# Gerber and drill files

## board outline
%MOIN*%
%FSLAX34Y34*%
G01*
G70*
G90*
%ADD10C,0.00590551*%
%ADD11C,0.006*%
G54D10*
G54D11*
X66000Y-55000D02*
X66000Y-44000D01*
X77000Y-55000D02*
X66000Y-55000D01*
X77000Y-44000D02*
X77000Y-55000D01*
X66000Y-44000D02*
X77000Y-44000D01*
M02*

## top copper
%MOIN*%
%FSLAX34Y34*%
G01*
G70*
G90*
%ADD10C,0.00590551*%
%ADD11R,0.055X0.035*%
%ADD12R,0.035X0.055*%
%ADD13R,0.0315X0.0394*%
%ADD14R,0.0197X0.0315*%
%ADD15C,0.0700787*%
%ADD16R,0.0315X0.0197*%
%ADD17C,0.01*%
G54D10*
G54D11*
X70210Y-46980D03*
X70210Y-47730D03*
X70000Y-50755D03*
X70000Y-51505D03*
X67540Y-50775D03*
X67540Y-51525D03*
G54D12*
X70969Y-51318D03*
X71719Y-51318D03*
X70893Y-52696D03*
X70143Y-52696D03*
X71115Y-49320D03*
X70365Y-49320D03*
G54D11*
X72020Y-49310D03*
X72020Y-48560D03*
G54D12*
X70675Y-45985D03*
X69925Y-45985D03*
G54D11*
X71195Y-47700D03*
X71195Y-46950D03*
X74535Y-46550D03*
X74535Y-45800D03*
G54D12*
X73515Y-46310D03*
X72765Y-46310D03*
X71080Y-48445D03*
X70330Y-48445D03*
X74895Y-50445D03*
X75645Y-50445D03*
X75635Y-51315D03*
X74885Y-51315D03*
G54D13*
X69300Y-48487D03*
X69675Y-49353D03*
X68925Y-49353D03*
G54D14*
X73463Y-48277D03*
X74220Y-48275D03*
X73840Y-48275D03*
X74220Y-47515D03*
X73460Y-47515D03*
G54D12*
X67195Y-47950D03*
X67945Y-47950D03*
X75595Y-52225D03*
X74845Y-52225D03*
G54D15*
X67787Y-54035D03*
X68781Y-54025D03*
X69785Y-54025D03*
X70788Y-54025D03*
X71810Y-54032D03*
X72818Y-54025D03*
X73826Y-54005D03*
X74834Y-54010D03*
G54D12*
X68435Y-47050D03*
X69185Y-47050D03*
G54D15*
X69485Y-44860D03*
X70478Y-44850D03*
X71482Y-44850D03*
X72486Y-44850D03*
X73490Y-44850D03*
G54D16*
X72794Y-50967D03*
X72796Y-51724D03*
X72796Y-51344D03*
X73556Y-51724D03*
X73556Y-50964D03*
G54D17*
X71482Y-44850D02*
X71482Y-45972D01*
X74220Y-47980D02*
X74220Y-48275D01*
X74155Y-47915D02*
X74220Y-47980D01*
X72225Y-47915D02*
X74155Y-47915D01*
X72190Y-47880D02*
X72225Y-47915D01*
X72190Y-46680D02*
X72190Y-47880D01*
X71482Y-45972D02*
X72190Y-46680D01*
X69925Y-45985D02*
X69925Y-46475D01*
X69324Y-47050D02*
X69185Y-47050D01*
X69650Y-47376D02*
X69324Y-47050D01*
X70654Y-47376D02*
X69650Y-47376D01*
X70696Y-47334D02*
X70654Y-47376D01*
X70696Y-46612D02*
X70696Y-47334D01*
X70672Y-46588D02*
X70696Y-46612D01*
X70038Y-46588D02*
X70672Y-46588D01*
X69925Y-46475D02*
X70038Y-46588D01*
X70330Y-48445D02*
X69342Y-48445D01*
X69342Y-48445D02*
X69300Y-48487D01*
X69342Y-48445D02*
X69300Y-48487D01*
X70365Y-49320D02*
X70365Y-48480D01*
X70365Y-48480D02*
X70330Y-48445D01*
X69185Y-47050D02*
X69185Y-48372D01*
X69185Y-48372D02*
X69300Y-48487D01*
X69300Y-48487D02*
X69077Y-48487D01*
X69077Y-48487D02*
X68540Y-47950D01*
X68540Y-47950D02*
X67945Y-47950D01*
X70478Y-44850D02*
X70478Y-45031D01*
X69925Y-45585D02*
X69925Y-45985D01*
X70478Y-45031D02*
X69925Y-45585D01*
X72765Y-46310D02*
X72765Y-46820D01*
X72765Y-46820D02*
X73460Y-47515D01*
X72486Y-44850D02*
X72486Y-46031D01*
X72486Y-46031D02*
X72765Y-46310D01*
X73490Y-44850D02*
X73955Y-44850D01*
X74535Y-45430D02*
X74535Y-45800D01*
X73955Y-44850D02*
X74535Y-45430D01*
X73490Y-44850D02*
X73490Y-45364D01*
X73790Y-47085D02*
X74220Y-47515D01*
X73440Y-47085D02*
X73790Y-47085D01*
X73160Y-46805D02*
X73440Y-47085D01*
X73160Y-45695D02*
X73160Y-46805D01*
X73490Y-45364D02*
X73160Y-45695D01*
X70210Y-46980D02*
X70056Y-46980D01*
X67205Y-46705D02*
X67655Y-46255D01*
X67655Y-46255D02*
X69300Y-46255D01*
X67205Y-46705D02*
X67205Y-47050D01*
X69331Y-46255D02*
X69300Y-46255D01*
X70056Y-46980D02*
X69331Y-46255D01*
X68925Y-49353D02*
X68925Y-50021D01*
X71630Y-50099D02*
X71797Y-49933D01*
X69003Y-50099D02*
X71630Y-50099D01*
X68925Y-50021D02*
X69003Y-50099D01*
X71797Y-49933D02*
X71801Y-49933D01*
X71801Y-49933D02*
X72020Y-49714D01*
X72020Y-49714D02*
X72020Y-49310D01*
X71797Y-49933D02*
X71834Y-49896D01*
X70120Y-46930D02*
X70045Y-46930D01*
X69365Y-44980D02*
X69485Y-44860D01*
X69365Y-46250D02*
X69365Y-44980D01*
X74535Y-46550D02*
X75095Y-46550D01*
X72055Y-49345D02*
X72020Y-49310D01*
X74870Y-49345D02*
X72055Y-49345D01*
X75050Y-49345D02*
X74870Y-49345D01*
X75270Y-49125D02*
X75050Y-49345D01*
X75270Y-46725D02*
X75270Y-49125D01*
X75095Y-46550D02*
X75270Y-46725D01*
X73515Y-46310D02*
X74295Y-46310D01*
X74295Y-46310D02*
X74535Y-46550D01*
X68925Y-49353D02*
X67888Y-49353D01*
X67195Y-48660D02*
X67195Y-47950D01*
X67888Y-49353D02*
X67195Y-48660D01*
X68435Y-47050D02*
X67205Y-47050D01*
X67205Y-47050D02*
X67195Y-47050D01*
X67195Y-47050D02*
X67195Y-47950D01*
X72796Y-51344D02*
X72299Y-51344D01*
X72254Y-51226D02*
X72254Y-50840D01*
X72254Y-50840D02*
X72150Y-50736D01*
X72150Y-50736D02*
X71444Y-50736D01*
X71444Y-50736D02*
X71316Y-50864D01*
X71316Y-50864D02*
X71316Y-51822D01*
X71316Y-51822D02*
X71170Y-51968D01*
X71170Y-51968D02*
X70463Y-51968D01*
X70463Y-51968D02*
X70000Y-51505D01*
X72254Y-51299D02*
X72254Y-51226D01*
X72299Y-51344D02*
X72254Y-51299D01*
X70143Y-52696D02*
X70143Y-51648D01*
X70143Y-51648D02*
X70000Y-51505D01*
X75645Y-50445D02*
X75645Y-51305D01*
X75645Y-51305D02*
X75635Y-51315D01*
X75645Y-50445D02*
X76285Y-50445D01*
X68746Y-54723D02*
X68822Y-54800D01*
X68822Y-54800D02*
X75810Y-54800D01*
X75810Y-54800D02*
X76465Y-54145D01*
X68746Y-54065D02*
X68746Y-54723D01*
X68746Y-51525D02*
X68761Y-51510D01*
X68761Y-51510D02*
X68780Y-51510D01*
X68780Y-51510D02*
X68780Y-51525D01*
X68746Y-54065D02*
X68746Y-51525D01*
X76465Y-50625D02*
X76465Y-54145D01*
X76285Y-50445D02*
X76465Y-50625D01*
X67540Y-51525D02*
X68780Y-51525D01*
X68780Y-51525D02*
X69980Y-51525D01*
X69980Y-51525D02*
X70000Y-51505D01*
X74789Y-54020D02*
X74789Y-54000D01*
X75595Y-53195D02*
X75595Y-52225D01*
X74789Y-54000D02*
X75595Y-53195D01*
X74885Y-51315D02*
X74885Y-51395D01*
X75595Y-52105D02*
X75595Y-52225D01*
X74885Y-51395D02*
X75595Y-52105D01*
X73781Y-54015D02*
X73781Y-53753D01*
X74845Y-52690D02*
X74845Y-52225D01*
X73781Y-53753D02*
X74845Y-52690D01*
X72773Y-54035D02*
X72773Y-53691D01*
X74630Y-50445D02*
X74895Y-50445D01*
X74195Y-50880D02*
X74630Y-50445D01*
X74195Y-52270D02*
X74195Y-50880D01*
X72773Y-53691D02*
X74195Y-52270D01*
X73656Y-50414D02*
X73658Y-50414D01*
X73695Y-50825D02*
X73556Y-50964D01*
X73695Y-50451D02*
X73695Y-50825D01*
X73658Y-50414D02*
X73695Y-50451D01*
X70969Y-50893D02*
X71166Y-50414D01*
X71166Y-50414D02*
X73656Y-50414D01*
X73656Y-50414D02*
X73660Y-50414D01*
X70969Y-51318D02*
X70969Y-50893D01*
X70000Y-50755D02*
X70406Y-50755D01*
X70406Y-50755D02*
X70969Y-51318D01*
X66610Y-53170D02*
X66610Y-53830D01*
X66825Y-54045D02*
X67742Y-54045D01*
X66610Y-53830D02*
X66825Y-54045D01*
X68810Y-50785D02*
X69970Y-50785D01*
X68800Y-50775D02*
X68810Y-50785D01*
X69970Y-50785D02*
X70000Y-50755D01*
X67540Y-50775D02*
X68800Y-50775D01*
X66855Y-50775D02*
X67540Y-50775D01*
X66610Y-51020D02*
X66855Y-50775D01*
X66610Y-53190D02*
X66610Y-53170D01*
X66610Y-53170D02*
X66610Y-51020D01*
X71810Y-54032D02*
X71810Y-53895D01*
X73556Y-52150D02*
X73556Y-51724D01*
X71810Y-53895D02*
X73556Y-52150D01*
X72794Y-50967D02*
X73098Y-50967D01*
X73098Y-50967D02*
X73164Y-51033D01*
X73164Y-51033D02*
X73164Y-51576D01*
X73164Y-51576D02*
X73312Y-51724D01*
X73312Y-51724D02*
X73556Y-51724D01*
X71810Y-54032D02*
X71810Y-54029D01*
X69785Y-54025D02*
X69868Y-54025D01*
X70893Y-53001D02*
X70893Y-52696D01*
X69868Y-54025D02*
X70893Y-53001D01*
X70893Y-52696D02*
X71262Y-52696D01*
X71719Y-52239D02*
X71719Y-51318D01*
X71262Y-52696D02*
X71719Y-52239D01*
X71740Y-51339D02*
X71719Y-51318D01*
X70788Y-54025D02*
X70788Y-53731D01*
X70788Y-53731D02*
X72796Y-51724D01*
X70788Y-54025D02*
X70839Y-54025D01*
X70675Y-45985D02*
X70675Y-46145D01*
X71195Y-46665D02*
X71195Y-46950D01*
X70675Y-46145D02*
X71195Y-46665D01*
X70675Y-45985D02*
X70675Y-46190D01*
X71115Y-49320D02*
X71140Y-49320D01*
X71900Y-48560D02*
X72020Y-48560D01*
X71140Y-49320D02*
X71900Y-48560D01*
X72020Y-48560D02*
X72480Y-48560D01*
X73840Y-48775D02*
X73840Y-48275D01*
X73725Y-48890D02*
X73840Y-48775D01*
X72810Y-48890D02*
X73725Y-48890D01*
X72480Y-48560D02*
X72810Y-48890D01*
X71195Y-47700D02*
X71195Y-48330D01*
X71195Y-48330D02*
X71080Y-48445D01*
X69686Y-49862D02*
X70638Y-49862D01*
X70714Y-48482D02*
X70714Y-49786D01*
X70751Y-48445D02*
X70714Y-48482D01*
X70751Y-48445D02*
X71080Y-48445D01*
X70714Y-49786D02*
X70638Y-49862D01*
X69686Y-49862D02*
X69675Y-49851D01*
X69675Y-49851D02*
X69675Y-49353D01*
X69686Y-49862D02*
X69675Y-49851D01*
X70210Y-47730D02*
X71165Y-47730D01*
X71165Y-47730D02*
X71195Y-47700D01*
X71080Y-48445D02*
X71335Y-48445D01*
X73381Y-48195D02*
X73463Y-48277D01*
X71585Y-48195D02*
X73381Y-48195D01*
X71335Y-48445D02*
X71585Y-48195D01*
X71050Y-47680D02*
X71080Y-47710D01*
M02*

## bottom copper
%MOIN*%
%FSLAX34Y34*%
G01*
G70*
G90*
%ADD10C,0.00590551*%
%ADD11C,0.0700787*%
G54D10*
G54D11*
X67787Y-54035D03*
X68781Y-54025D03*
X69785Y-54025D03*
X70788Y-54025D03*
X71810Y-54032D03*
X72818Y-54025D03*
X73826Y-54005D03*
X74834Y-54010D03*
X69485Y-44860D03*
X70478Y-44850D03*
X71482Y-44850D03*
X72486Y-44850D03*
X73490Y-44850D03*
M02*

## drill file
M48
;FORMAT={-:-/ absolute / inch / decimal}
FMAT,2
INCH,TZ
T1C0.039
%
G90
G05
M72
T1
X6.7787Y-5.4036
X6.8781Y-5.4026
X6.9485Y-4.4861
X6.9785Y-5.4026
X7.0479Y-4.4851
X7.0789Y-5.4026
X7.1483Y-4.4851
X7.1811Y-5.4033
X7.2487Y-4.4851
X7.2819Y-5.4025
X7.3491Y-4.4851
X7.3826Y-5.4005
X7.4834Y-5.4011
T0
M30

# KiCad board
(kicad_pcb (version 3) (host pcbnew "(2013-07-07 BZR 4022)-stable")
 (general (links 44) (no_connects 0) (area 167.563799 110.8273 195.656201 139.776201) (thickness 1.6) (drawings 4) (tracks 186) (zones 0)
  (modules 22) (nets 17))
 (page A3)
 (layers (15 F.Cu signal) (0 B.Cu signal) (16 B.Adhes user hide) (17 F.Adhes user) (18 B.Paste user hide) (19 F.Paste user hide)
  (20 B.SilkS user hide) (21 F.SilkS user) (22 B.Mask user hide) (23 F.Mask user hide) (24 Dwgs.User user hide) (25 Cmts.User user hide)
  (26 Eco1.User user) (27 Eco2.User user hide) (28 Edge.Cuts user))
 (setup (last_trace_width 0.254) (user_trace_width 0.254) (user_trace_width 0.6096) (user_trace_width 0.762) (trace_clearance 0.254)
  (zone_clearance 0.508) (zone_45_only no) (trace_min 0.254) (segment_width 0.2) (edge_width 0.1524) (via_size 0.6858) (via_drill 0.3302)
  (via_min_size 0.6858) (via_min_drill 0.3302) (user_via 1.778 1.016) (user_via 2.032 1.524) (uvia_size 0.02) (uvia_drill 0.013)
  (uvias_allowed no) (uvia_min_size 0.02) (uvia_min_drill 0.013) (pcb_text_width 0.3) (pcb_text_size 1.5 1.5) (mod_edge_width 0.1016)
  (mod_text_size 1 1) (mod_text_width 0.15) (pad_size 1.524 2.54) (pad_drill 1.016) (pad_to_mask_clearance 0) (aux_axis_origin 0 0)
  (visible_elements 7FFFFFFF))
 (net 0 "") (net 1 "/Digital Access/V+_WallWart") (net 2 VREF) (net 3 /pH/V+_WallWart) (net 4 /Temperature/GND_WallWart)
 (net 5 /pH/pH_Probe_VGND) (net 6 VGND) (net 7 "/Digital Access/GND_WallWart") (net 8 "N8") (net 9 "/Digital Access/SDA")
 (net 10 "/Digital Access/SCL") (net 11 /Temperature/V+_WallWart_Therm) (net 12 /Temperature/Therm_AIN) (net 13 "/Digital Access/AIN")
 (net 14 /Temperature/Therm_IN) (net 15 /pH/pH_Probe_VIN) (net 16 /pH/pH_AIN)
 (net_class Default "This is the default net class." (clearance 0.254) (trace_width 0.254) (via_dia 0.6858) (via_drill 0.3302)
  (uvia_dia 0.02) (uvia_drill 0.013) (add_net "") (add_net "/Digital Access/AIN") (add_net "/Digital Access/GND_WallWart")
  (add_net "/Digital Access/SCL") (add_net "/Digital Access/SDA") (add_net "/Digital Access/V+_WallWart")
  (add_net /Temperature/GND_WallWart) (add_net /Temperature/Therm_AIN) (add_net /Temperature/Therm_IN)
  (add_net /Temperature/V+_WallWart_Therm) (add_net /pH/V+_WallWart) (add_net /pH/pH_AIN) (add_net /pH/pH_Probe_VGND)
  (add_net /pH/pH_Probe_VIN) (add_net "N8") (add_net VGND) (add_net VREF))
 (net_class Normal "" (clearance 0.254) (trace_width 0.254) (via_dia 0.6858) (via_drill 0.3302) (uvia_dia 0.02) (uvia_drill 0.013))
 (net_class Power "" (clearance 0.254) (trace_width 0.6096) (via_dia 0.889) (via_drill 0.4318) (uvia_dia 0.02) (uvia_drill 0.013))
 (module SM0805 (layer F.Cu) (at 178.3334 120.2817 270)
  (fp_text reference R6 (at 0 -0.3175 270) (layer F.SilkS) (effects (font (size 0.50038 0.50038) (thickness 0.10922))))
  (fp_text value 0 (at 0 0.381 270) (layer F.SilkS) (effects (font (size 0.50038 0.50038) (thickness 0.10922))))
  (pad 1 smd rect (at -0.9525 0 270) (size 0.889 1.397) (layers F.Cu F.Paste F.Mask) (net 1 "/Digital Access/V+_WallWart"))
  (pad 2 smd rect (at 0.9525 0 270) (size 0.889 1.397) (layers F.Cu F.Paste F.Mask) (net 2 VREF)))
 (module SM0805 (layer F.Cu) (at 177.8 129.8702 270)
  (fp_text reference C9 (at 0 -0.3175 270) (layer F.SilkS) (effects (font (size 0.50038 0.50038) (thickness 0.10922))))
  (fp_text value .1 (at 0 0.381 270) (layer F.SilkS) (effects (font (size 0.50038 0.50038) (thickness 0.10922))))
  (pad 1 smd rect (at -0.9525 0 270) (size 0.889 1.397) (layers F.Cu F.Paste F.Mask) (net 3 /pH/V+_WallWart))
  (pad 2 smd rect (at 0.9525 0 270) (size 0.889 1.397) (layers F.Cu F.Paste F.Mask) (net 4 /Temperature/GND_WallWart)))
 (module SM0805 (layer F.Cu) (at 171.5516 129.921 270)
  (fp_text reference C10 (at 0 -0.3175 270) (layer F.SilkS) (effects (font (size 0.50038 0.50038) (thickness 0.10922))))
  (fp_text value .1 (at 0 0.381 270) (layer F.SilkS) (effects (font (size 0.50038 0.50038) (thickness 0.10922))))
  (pad 1 smd rect (at -0.9525 0 270) (size 0.889 1.397) (layers F.Cu F.Paste F.Mask) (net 3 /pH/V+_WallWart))
  (pad 2 smd rect (at 0.9525 0 270) (size 0.889 1.397) (layers F.Cu F.Paste F.Mask) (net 4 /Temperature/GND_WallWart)))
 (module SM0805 (layer F.Cu) (at 181.21376 130.34772)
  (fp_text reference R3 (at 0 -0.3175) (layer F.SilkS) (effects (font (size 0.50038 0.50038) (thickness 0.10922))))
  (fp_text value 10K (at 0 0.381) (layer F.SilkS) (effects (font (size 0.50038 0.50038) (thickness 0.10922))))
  (pad 1 smd rect (at -0.9525 0) (size 0.889 1.397) (layers F.Cu F.Paste F.Mask) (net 3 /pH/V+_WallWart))
  (pad 2 smd rect (at 0.9525 0) (size 0.889 1.397) (layers F.Cu F.Paste F.Mask) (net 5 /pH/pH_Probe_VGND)))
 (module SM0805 (layer F.Cu) (at 179.11572 133.84784 180)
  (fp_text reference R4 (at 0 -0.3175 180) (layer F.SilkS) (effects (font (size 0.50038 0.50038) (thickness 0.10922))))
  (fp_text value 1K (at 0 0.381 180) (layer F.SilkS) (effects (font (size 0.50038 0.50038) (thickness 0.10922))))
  (pad 1 smd rect (at -0.9525 0 180) (size 0.889 1.397) (layers F.Cu F.Paste F.Mask) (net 5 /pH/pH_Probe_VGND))
  (pad 2 smd rect (at 0.9525 0 180) (size 0.889 1.397) (layers F.Cu F.Paste F.Mask) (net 4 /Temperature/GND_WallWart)))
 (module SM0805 (layer F.Cu) (at 179.6796 125.2728 180)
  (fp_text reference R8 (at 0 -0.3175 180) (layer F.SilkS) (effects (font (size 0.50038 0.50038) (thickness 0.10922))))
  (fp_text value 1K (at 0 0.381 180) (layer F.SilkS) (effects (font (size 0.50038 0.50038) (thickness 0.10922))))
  (pad 1 smd rect (at -0.9525 0 180) (size 0.889 1.397) (layers F.Cu F.Paste F.Mask) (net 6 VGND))
  (pad 2 smd rect (at 0.9525 0 180) (size 0.889 1.397) (layers F.Cu F.Paste F.Mask) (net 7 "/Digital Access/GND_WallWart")))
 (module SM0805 (layer F.Cu) (at 182.9308 124.2949 90)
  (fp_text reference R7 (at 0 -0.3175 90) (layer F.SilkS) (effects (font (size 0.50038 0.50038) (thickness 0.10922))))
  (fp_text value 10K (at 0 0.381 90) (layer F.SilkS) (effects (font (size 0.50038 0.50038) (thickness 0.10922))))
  (pad 1 smd rect (at -0.9525 0 90) (size 0.889 1.397) (layers F.Cu F.Paste F.Mask) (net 1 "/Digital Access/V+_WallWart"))
  (pad 2 smd rect (at 0.9525 0 90) (size 0.889 1.397) (layers F.Cu F.Paste F.Mask) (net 6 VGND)))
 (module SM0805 (layer F.Cu) (at 178.562 116.8019 180)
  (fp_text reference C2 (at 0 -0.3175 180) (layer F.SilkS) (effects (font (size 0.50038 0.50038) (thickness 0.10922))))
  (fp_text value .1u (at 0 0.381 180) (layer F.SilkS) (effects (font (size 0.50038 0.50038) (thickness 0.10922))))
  (pad 1 smd rect (at -0.9525 0 180) (size 0.889 1.397) (layers F.Cu F.Paste F.Mask) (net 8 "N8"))
  (pad 2 smd rect (at 0.9525 0 180) (size 0.889 1.397) (layers F.Cu F.Paste F.Mask) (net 7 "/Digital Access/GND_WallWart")))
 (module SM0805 (layer F.Cu) (at 180.8353 120.2055 90)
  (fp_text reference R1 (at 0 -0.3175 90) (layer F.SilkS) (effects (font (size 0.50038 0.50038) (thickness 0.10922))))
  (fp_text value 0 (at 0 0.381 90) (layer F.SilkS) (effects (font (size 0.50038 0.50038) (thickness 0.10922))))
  (pad 1 smd rect (at -0.9525 0 90) (size 0.889 1.397) (layers F.Cu F.Paste F.Mask) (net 2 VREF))
  (pad 2 smd rect (at 0.9525 0 90) (size 0.889 1.397) (layers F.Cu F.Paste F.Mask) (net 8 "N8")))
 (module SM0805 (layer F.Cu) (at 189.3189 117.2845 90)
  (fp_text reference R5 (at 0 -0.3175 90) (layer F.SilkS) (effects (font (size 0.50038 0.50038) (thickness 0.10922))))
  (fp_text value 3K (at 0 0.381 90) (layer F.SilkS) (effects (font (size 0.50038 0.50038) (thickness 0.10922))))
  (pad 1 smd rect (at -0.9525 0 90) (size 0.889 1.397) (layers F.Cu F.Paste F.Mask) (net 1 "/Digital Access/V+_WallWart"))
  (pad 2 smd rect (at 0.9525 0 90) (size 0.889 1.397) (layers F.Cu F.Paste F.Mask) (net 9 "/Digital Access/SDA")))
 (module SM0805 (layer F.Cu) (at 185.7756 117.6274 180)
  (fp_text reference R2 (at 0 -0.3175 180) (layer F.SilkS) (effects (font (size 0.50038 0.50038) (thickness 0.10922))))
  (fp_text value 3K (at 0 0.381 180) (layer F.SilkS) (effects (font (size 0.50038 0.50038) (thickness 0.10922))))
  (pad 1 smd rect (at -0.9525 0 180) (size 0.889 1.397) (layers F.Cu F.Paste F.Mask) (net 1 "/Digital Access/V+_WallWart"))
  (pad 2 smd rect (at 0.9525 0 180) (size 0.889 1.397) (layers F.Cu F.Paste F.Mask) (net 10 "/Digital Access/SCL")))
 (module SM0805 (layer F.Cu) (at 179.5907 123.0503 180)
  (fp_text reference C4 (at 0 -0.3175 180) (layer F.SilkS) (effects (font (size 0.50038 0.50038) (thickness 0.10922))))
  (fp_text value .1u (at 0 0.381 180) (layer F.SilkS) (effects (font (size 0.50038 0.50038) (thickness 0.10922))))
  (pad 1 smd rect (at -0.9525 0 180) (size 0.889 1.397) (layers F.Cu F.Paste F.Mask) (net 2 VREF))
  (pad 2 smd rect (at 0.9525 0 180) (size 0.889 1.397) (layers F.Cu F.Paste F.Mask) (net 7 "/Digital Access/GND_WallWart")))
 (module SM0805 (layer F.Cu) (at 191.1858 128.1303)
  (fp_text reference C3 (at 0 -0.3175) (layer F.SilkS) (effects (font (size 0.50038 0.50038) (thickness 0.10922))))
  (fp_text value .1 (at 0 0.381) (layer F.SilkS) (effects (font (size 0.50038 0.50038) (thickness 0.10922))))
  (pad 1 smd rect (at -0.9525 0) (size 0.889 1.397) (layers F.Cu F.Paste F.Mask) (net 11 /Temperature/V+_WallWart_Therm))
  (pad 2 smd rect (at 0.9525 0) (size 0.889 1.397) (layers F.Cu F.Paste F.Mask) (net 4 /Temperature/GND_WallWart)))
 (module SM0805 (layer F.Cu) (at 191.1604 130.3401 180)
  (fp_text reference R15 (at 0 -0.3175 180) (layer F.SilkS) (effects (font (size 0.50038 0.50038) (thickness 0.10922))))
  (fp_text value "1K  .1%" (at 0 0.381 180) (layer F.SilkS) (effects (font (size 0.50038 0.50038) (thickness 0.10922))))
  (pad 1 smd rect (at -0.9525 0 180) (size 0.889 1.397) (layers F.Cu F.Paste F.Mask) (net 4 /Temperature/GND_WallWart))
  (pad 2 smd rect (at 0.9525 0 180) (size 0.889 1.397) (layers F.Cu F.Paste F.Mask) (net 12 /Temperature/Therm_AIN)))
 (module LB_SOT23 (layer F.Cu) (at 176.022 124.2568)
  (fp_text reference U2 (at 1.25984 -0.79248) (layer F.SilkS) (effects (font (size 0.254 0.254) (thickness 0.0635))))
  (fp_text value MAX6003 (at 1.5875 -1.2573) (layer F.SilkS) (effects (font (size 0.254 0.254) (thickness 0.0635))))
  (pad 3 smd rect (at 0 -1.09982) (size 0.8001 1.00076) (layers F.Cu F.Paste F.Mask) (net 7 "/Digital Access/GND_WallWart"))
  (pad 2 smd rect (at 0.9525 1.09982) (size 0.8001 1.00076) (layers F.Cu F.Paste F.Mask) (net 2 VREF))
  (pad 1 smd rect (at -0.9525 1.09982) (size 0.8001 1.00076) (layers F.Cu F.Paste F.Mask) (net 1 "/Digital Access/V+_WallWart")))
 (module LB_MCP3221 (layer F.Cu) (at 186.5884 122.5423)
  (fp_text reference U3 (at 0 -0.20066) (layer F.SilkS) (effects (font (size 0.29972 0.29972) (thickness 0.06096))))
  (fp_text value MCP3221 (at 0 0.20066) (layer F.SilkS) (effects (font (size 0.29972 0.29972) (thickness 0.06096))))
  (pad 1 smd rect (at 0.00762 0.08128) (size 0.50038 0.8001) (layers F.Cu F.Paste F.Mask) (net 2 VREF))
  (pad 3 smd rect (at 1.9304 0.0762) (size 0.50038 0.8001) (layers F.Cu F.Paste F.Mask) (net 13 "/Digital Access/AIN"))
  (pad 2 smd rect (at 0.9652 0.0762) (size 0.50038 0.8001) (layers F.Cu F.Paste F.Mask) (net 6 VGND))
  (pad 4 smd rect (at 1.9304 -1.8542) (size 0.50038 0.8001) (layers F.Cu F.Paste F.Mask) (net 9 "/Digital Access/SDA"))
  (pad 5 smd rect (at 0 -1.8542) (size 0.50038 0.8001) (layers F.Cu F.Paste F.Mask) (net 10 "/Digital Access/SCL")))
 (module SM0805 (layer F.Cu) (at 171.6278 121.793)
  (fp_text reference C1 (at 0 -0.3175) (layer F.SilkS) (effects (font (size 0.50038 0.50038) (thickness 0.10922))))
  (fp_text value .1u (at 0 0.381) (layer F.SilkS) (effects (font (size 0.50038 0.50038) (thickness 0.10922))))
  (pad 1 smd rect (at -0.9525 0) (size 0.889 1.397) (layers F.Cu F.Paste F.Mask) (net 1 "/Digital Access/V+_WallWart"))
  (pad 2 smd rect (at 0.9525 0) (size 0.889 1.397) (layers F.Cu F.Paste F.Mask) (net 7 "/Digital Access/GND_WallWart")))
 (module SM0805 (layer F.Cu) (at 191.0588 132.6515 180)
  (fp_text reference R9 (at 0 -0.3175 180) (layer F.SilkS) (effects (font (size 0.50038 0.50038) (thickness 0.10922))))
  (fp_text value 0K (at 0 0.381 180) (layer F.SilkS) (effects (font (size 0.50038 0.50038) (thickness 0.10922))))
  (pad 1 smd rect (at -0.9525 0 180) (size 0.889 1.397) (layers F.Cu F.Paste F.Mask) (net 12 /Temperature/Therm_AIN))
  (pad 2 smd rect (at 0.9525 0 180) (size 0.889 1.397) (layers F.Cu F.Paste F.Mask) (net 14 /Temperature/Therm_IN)))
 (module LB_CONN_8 (layer F.Cu) (at 177.2793 137.2108)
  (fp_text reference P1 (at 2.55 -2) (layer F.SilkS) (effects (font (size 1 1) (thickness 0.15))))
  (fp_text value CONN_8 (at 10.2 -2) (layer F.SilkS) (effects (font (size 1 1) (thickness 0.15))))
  (pad 1 thru_hole circle (at -5.1 0.04) (size 1.78 1.78) (drill 1) (layers *.Cu *.Mask F.SilkS) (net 3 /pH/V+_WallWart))
  (pad 2 thru_hole circle (at -2.5754 0.0146) (size 1.78 1.78) (drill 1) (layers *.Cu *.Mask F.SilkS) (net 4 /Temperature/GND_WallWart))
  (pad 3 thru_hole circle (at -0.0254 0.0146) (size 1.78 1.78) (drill 1) (layers *.Cu *.Mask F.SilkS) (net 5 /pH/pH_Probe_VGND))
  (pad 4 thru_hole circle (at 2.5246 0.0146) (size 1.78 1.78) (drill 1) (layers *.Cu *.Mask F.SilkS) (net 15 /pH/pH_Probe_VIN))
  (pad 5 thru_hole circle (at 5.12 0.033) (size 1.78 1.78) (drill 1) (layers *.Cu *.Mask F.SilkS) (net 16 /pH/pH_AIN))
  (pad 6 thru_hole circle (at 7.68 0.013) (size 1.78 1.78) (drill 1) (layers *.Cu *.Mask F.SilkS) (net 11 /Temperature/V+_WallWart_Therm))
  (pad 7 thru_hole circle (at 10.24 -0.038) (size 1.78 1.78) (drill 1) (layers *.Cu *.Mask F.SilkS) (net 14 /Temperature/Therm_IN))
  (pad 8 thru_hole circle (at 12.8 -0.023) (size 1.78 1.78) (drill 1) (layers *.Cu *.Mask F.SilkS) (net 12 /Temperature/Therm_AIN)))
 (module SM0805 (layer F.Cu) (at 174.7774 119.507)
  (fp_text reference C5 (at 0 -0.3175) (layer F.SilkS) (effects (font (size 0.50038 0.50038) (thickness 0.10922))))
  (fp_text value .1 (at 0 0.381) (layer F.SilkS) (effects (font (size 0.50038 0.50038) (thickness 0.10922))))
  (pad 1 smd rect (at -0.9525 0) (size 0.889 1.397) (layers F.Cu F.Paste F.Mask) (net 1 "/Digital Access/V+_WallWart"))
  (pad 2 smd rect (at 0.9525 0) (size 0.889 1.397) (layers F.Cu F.Paste F.Mask) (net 7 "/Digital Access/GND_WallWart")))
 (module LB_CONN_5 (layer F.Cu) (at 176.4919 113.9063)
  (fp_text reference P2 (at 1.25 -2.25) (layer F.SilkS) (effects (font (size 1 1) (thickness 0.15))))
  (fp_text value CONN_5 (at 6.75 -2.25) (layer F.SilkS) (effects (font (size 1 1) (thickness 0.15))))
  (pad 1 thru_hole circle (at 0 0.04) (size 1.78 1.78) (drill 1) (layers *.Cu *.Mask F.SilkS) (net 1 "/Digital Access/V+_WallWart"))
  (pad 2 thru_hole circle (at 2.5246 0.0146) (size 1.78 1.78) (drill 1) (layers *.Cu *.Mask F.SilkS) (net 7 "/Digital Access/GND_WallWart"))
  (pad 3 thru_hole circle (at 5.0746 0.0146) (size 1.78 1.78) (drill 1) (layers *.Cu *.Mask F.SilkS) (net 13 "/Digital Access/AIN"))
  (pad 4 thru_hole circle (at 7.6246 0.0146) (size 1.78 1.78) (drill 1) (layers *.Cu *.Mask F.SilkS) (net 10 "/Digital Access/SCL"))
  (pad 5 thru_hole circle (at 10.1746 0.0146) (size 1.78 1.78) (drill 1) (layers *.Cu *.Mask F.SilkS) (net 9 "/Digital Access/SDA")))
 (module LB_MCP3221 (layer F.Cu) (at 184.97804 129.44856 270)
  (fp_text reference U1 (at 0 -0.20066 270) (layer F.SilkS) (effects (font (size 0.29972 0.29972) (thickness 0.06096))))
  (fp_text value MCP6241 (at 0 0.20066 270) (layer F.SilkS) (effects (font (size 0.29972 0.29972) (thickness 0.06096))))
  (pad 1 smd rect (at 0.00762 0.08128 270) (size 0.50038 0.8001) (layers F.Cu F.Paste F.Mask) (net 16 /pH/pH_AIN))
  (pad 3 smd rect (at 1.9304 0.0762 270) (size 0.50038 0.8001) (layers F.Cu F.Paste F.Mask) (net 15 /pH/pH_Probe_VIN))
  (pad 2 smd rect (at 0.9652 0.0762 270) (size 0.50038 0.8001) (layers F.Cu F.Paste F.Mask) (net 4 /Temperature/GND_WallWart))
  (pad 4 smd rect (at 1.9304 -1.8542 270) (size 0.50038 0.8001) (layers F.Cu F.Paste F.Mask) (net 16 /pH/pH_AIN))
  (pad 5 smd rect (at 0 -1.8542 270) (size 0.50038 0.8001) (layers F.Cu F.Paste F.Mask) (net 3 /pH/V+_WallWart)))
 (gr_line (start 167.64 139.7) (end 167.64 111.76) (angle 90) (layer Edge.Cuts) (width 0.1524))
 (gr_line (start 195.58 139.7) (end 167.64 139.7) (angle 90) (layer Edge.Cuts) (width 0.1524))
 (gr_line (start 195.58 111.76) (end 195.58 139.7) (angle 90) (layer Edge.Cuts) (width 0.1524))
 (gr_line (start 167.64 111.76) (end 195.58 111.76) (angle 90) (layer Edge.Cuts) (width 0.1524))
 (segment (start 181.5665 113.9209) (end 181.5665 116.7711) (width 0.254) (layer F.Cu) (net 13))
 (segment (start 188.5188 121.8692) (end 188.5188 122.6185) (width 0.254) (layer F.Cu) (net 13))
 (segment (start 188.3537 121.7041) (end 188.5188 121.8692) (width 0.254) (layer F.Cu) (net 13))
 (segment (start 183.4515 121.7041) (end 188.3537 121.7041) (width 0.254) (layer F.Cu) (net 13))
 (segment (start 183.3626 121.6152) (end 183.4515 121.7041) (width 0.254) (layer F.Cu) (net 13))
 (segment (start 183.3626 118.5672) (end 183.3626 121.6152) (width 0.254) (layer F.Cu) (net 13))
 (segment (start 181.5665 116.7711) (end 183.3626 118.5672) (width 0.254) (layer F.Cu) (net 13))
 (segment (start 177.6095 116.8019) (end 177.6095 118.0465) (width 0.254) (layer F.Cu) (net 7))
 (segment (start 176.08296 119.507) (end 175.7299 119.507) (width 0.254) (layer F.Cu) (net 7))
 (segment (start 176.911 120.33504) (end 176.08296 119.507) (width 0.254) (layer F.Cu) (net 7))
 (segment (start 179.46116 120.33504) (end 176.911 120.33504) (width 0.254) (layer F.Cu) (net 7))
 (segment (start 179.56784 120.22836) (end 179.46116 120.33504) (width 0.254) (layer F.Cu) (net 7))
 (segment (start 179.56784 118.39448) (end 179.56784 120.22836) (width 0.254) (layer F.Cu) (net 7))
 (segment (start 179.50688 118.33352) (end 179.56784 118.39448) (width 0.254) (layer F.Cu) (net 7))
 (segment (start 177.89652 118.33352) (end 179.50688 118.33352) (width 0.254) (layer F.Cu) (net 7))
 (segment (start 177.6095 118.0465) (end 177.89652 118.33352) (width 0.254) (layer F.Cu) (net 7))
 (segment (start 178.6382 123.0503) (end 176.12868 123.0503) (width 0.254) (layer F.Cu) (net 7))
 (segment (start 176.12868 123.0503) (end 176.022 123.15698) (width 0.254) (layer F.Cu) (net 7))
 (segment (start 176.12868 123.0503) (end 176.022 123.15698) (width 0.254) (layer F.Cu) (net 7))
 (segment (start 178.7271 125.2728) (end 178.7271 123.1392) (width 0.254) (layer F.Cu) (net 7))
 (segment (start 178.7271 123.1392) (end 178.6382 123.0503) (width 0.254) (layer F.Cu) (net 7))
 (segment (start 175.7299 119.507) (end 175.7299 122.86488) (width 0.254) (layer F.Cu) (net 7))
 (segment (start 175.7299 122.86488) (end 176.022 123.15698) (width 0.254) (layer F.Cu) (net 7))
 (segment (start 176.022 123.15698) (end 175.45558 123.15698) (width 0.254) (layer F.Cu) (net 7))
 (segment (start 175.45558 123.15698) (end 174.0916 121.793) (width 0.254) (layer F.Cu) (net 7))
 (segment (start 174.0916 121.793) (end 172.5803 121.793) (width 0.254) (layer F.Cu) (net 7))
 (segment (start 179.0165 113.9209) (end 179.0165 114.3789) (width 0.254) (layer F.Cu) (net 7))
 (segment (start 177.6095 115.7859) (end 177.6095 116.8019) (width 0.254) (layer F.Cu) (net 7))
 (segment (start 179.0165 114.3789) (end 177.6095 115.7859) (width 0.254) (layer F.Cu) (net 7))
 (segment (start 184.8231 117.6274) (end 184.8231 118.9228) (width 0.254) (layer F.Cu) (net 10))
 (segment (start 184.8231 118.9228) (end 186.5884 120.6881) (width 0.254) (layer F.Cu) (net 10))
 (segment (start 184.1165 113.9209) (end 184.1165 116.9208) (width 0.254) (layer F.Cu) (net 10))
 (segment (start 184.1165 116.9208) (end 184.8231 117.6274) (width 0.254) (layer F.Cu) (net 10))
 (segment (start 186.6665 113.9209) (end 187.8476 113.9209) (width 0.254) (layer F.Cu) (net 9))
 (segment (start 189.3189 115.3922) (end 189.3189 116.332) (width 0.254) (layer F.Cu) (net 9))
 (segment (start 187.8476 113.9209) (end 189.3189 115.3922) (width 0.254) (layer F.Cu) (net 9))
 (segment (start 186.6665 113.9209) (end 186.6665 115.2252) (width 0.254) (layer F.Cu) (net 9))
 (segment (start 187.4266 119.5959) (end 188.5188 120.6881) (width 0.254) (layer F.Cu) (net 9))
 (segment (start 186.5376 119.5959) (end 187.4266 119.5959) (width 0.254) (layer F.Cu) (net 9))
 (segment (start 185.8264 118.8847) (end 186.5376 119.5959) (width 0.254) (layer F.Cu) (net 9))
 (segment (start 185.8264 116.0653) (end 185.8264 118.8847) (width 0.254) (layer F.Cu) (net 9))
 (segment (start 186.6665 115.2252) (end 185.8264 116.0653) (width 0.254) (layer F.Cu) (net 9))
 (segment (start 178.3334 119.3292) (end 177.94224 119.3292) (width 0.254) (layer F.Cu) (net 1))
 (segment (start 170.7007 118.6307) (end 171.8437 117.4877) (width 0.254) (layer F.Cu) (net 1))
 (segment (start 171.8437 117.4877) (end 176.022 117.4877) (width 0.254) (layer F.Cu) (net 1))
 (segment (start 170.7007 118.6307) (end 170.7007 119.507) (width 0.254) (layer F.Cu) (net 1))
 (segment (start 176.10074 117.4877) (end 176.022 117.4877) (width 0.254) (layer F.Cu) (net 1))
 (segment (start 177.94224 119.3292) (end 176.10074 117.4877) (width 0.254) (layer F.Cu) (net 1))
 (segment (start 175.0695 125.35662) (end 175.0695 127.05334) (width 0.254) (layer F.Cu) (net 1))
 (segment (start 181.940202 127.253998) (end 182.36438 126.82982) (width 0.254) (layer F.Cu) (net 1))
 (segment (start 175.270158 127.253998) (end 181.940202 127.253998) (width 0.254) (layer F.Cu) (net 1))
 (segment (start 175.0695 127.05334) (end 175.270158 127.253998) (width 0.254) (layer F.Cu) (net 1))
 (segment (start 182.36438 126.82982) (end 182.37454 126.82982) (width 0.254) (layer F.Cu) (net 1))
 (segment (start 182.37454 126.82982) (end 182.9308 126.27356) (width 0.254) (layer F.Cu) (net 1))
 (segment (start 182.9308 126.27356) (end 182.9308 125.2474) (width 0.254) (layer F.Cu) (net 1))
 (segment (start 182.36438 126.82982) (end 182.45836 126.73584) (width 0.254) (layer F.Cu) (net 1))
 (segment (start 178.1048 119.2022) (end 177.9143 119.2022) (width 0.254) (layer F.Cu) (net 1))
 (segment (start 176.1871 114.2511) (end 176.4919 113.9463) (width 0.254) (layer F.Cu) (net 1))
 (segment (start 176.1871 117.475) (end 176.1871 114.2511) (width 0.254) (layer F.Cu) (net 1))
 (segment (start 189.3189 118.237) (end 190.7413 118.237) (width 0.254) (layer F.Cu) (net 1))
 (segment (start 183.0197 125.3363) (end 182.9308 125.2474) (width 0.254) (layer F.Cu) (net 1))
 (segment (start 190.1698 125.3363) (end 183.0197 125.3363) (width 0.254) (layer F.Cu) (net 1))
 (segment (start 190.627 125.3363) (end 190.1698 125.3363) (width 0.254) (layer F.Cu) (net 1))
 (segment (start 191.1858 124.7775) (end 190.627 125.3363) (width 0.254) (layer F.Cu) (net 1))
 (segment (start 191.1858 118.6815) (end 191.1858 124.7775) (width 0.254) (layer F.Cu) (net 1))
 (segment (start 190.7413 118.237) (end 191.1858 118.6815) (width 0.254) (layer F.Cu) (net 1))
 (segment (start 186.7281 117.6274) (end 188.7093 117.6274) (width 0.254) (layer F.Cu) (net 1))
 (segment (start 188.7093 117.6274) (end 189.3189 118.237) (width 0.254) (layer F.Cu) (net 1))
 (segment (start 175.0695 125.35662) (end 172.43552 125.35662) (width 0.254) (layer F.Cu) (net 1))
 (segment (start 170.6753 123.5964) (end 170.6753 121.793) (width 0.254) (layer F.Cu) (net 1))
 (segment (start 172.43552 125.35662) (end 170.6753 123.5964) (width 0.254) (layer F.Cu) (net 1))
 (segment (start 173.8249 119.507) (end 170.7007 119.507) (width 0.254) (layer F.Cu) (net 1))
 (segment (start 170.7007 119.507) (end 170.6753 119.507) (width 0.254) (layer F.Cu) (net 1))
 (segment (start 170.6753 119.507) (end 170.6753 121.793) (width 0.254) (layer F.Cu) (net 1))
 (segment (start 184.90184 130.41376) (end 183.63946 130.41376) (width 0.254) (layer F.Cu) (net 4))
 (segment (start 183.52516 130.11404) (end 183.52516 129.1336) (width 0.254) (layer F.Cu) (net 4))
 (segment (start 183.52516 129.1336) (end 183.261 128.86944) (width 0.254) (layer F.Cu) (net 4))
 (segment (start 183.261 128.86944) (end 181.46776 128.86944) (width 0.254) (layer F.Cu) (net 4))
 (segment (start 181.46776 128.86944) (end 181.14264 129.19456) (width 0.254) (layer F.Cu) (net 4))
 (segment (start 181.14264 129.19456) (end 181.14264 131.62788) (width 0.254) (layer F.Cu) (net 4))
 (segment (start 181.14264 131.62788) (end 180.7718 131.99872) (width 0.254) (layer F.Cu) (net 4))
 (segment (start 180.7718 131.99872) (end 178.97602 131.99872) (width 0.254) (layer F.Cu) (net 4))
 (segment (start 178.97602 131.99872) (end 177.8 130.8227) (width 0.254) (layer F.Cu) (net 4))
 (segment (start 183.52516 130.29946) (end 183.52516 130.11404) (width 0.254) (layer F.Cu) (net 4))
 (segment (start 183.63946 130.41376) (end 183.52516 130.29946) (width 0.254) (layer F.Cu) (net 4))
 (segment (start 178.16322 133.84784) (end 178.16322 131.18592) (width 0.254) (layer F.Cu) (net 4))
 (segment (start 178.16322 131.18592) (end 177.8 130.8227) (width 0.254) (layer F.Cu) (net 4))
 (segment (start 192.1383 128.1303) (end 192.1383 130.3147) (width 0.254) (layer F.Cu) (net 4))
 (segment (start 192.1383 130.3147) (end 192.1129 130.3401) (width 0.254) (layer F.Cu) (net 4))
 (segment (start 192.1383 128.1303) (end 193.7639 128.1303) (width 0.254) (layer F.Cu) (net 4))
 (segment (start 174.615 138.9988) (end 174.8082 139.192) (width 0.254) (layer F.Cu) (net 4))
 (segment (start 174.8082 139.192) (end 192.5574 139.192) (width 0.254) (layer F.Cu) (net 4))
 (segment (start 192.5574 139.192) (end 194.2211 137.5283) (width 0.254) (layer F.Cu) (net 4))
 (segment (start 174.615 137.327) (end 174.615 138.9988) (width 0.254) (layer F.Cu) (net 4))
 (segment (start 174.615 130.8735) (end 174.6531 130.8354) (width 0.254) (layer F.Cu) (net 4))
 (segment (start 174.6531 130.8354) (end 174.7012 130.8354) (width 0.254) (layer F.Cu) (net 4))
 (segment (start 174.7012 130.8354) (end 174.7012 130.8735) (width 0.254) (layer F.Cu) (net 4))
 (segment (start 174.615 137.327) (end 174.615 130.8735) (width 0.254) (layer F.Cu) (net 4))
 (segment (start 194.2211 128.5875) (end 194.2211 137.5283) (width 0.254) (layer F.Cu) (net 4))
 (segment (start 193.7639 128.1303) (end 194.2211 128.5875) (width 0.254) (layer F.Cu) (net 4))
 (segment (start 171.5516 130.8735) (end 174.7012 130.8735) (width 0.254) (layer F.Cu) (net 4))
 (segment (start 174.7012 130.8735) (end 177.7492 130.8735) (width 0.254) (layer F.Cu) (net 4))
 (segment (start 177.7492 130.8735) (end 177.8 130.8227) (width 0.254) (layer F.Cu) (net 4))
 (segment (start 189.965 137.2132) (end 189.965 137.1616) (width 0.254) (layer F.Cu) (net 12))
 (segment (start 192.0113 135.1153) (end 192.0113 132.6515) (width 0.254) (layer F.Cu) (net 12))
 (segment (start 189.965 137.1616) (end 192.0113 135.1153) (width 0.254) (layer F.Cu) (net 12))
 (segment (start 190.2079 130.3401) (end 190.2079 130.5433) (width 0.254) (layer F.Cu) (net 12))
 (segment (start 192.0113 132.3467) (end 192.0113 132.6515) (width 0.254) (layer F.Cu) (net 12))
 (segment (start 190.2079 130.5433) (end 192.0113 132.3467) (width 0.254) (layer F.Cu) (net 12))
 (segment (start 187.405 137.1982) (end 187.405 136.5339) (width 0.254) (layer F.Cu) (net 14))
 (segment (start 190.1063 133.8326) (end 190.1063 132.6515) (width 0.254) (layer F.Cu) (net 14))
 (segment (start 187.405 136.5339) (end 190.1063 133.8326) (width 0.254) (layer F.Cu) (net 14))
 (segment (start 184.845 137.2492) (end 184.845 136.3761) (width 0.254) (layer F.Cu) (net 11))
 (segment (start 189.5602 128.1303) (end 190.2333 128.1303) (width 0.254) (layer F.Cu) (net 11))
 (segment (start 188.4553 129.2352) (end 189.5602 128.1303) (width 0.254) (layer F.Cu) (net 11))
 (segment (start 188.4553 132.7658) (end 188.4553 129.2352) (width 0.254) (layer F.Cu) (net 11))
 (segment (start 184.845 136.3761) (end 188.4553 132.7658) (width 0.254) (layer F.Cu) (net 11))
 (segment (start 187.08624 128.05156) (end 187.09132 128.05156) (width 0.254) (layer F.Cu) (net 3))
 (segment (start 187.1853 129.0955) (end 186.83224 129.44856) (width 0.254) (layer F.Cu) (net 3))
 (segment (start 187.1853 128.14554) (end 187.1853 129.0955) (width 0.254) (layer F.Cu) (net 3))
 (segment (start 187.09132 128.05156) (end 187.1853 128.14554) (width 0.254) (layer F.Cu) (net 3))
 (segment (start 180.26126 129.26822) (end 180.76164 128.05156) (width 0.254) (layer F.Cu) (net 3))
 (segment (start 180.76164 128.05156) (end 187.08624 128.05156) (width 0.254) (layer F.Cu) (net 3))
 (segment (start 187.08624 128.05156) (end 187.0964 128.05156) (width 0.254) (layer F.Cu) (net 3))
 (segment (start 180.26126 130.34772) (end 180.26126 129.26822) (width 0.254) (layer F.Cu) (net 3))
 (segment (start 177.8 128.9177) (end 178.83124 128.9177) (width 0.254) (layer F.Cu) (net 3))
 (segment (start 178.83124 128.9177) (end 180.26126 130.34772) (width 0.254) (layer F.Cu) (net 3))
 (segment (start 169.1894 135.0518) (end 169.1894 136.7282) (width 0.254) (layer F.Cu) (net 3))
 (segment (start 169.7374 137.2762) (end 172.065 137.2762) (width 0.254) (layer F.Cu) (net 3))
 (segment (start 169.1894 136.7282) (end 169.7374 137.2762) (width 0.254) (layer F.Cu) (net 3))
 (segment (start 174.7774 128.9939) (end 177.7238 128.9939) (width 0.254) (layer F.Cu) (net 3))
 (segment (start 174.752 128.9685) (end 174.7774 128.9939) (width 0.254) (layer F.Cu) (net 3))
 (segment (start 177.7238 128.9939) (end 177.8 128.9177) (width 0.254) (layer F.Cu) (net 3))
 (segment (start 171.5516 128.9685) (end 174.752 128.9685) (width 0.254) (layer F.Cu) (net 3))
 (segment (start 169.8117 128.9685) (end 171.5516 128.9685) (width 0.254) (layer F.Cu) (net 3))
 (segment (start 169.1894 129.5908) (end 169.8117 128.9685) (width 0.254) (layer F.Cu) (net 3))
 (segment (start 169.1894 135.1026) (end 169.1894 135.0518) (width 0.254) (layer F.Cu) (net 3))
 (segment (start 169.1894 135.0518) (end 169.1894 129.5908) (width 0.254) (layer F.Cu) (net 3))
 (segment (start 182.3993 137.2438) (end 182.3993 136.89394) (width 0.254) (layer F.Cu) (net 16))
 (segment (start 186.83224 132.461) (end 186.83224 131.37896) (width 0.254) (layer F.Cu) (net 16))
 (segment (start 182.3993 136.89394) (end 186.83224 132.461) (width 0.254) (layer F.Cu) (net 16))
 (segment (start 184.89676 129.45618) (end 185.66892 129.45618) (width 0.254) (layer F.Cu) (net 16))
 (segment (start 185.66892 129.45618) (end 185.83656 129.62382) (width 0.254) (layer F.Cu) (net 16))
 (segment (start 185.83656 129.62382) (end 185.83656 131.00304) (width 0.254) (layer F.Cu) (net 16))
 (segment (start 185.83656 131.00304) (end 186.21248 131.37896) (width 0.254) (layer F.Cu) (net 16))
 (segment (start 186.21248 131.37896) (end 186.83224 131.37896) (width 0.254) (layer F.Cu) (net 16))
 (segment (start 182.3993 137.2438) (end 182.3993 137.2343) (width 0.254) (layer F.Cu) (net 16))
 (segment (start 177.2539 137.2254) (end 177.46536 137.2254) (width 0.254) (layer F.Cu) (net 5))
 (segment (start 180.06822 134.62254) (end 180.06822 133.84784) (width 0.254) (layer F.Cu) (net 5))
 (segment (start 177.46536 137.2254) (end 180.06822 134.62254) (width 0.254) (layer F.Cu) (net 5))
 (segment (start 180.06822 133.84784) (end 181.00548 133.84784) (width 0.254) (layer F.Cu) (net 5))
 (segment (start 182.16626 132.68706) (end 182.16626 130.34772) (width 0.254) (layer F.Cu) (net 5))
 (segment (start 181.00548 133.84784) (end 182.16626 132.68706) (width 0.254) (layer F.Cu) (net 5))
 (segment (start 182.2196 130.40106) (end 182.16626 130.34772) (width 0.254) (layer F.Cu) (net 5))
 (segment (start 179.8039 137.2254) (end 179.8039 136.4769) (width 0.254) (layer F.Cu) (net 15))
 (segment (start 179.8039 136.4769) (end 184.90184 131.37896) (width 0.254) (layer F.Cu) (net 15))
 (segment (start 179.8039 137.2254) (end 179.9317 137.2254) (width 0.254) (layer F.Cu) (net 15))
 (segment (start 179.5145 116.8019) (end 179.5145 117.2083) (width 0.254) (layer F.Cu) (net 8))
 (segment (start 180.8353 118.5291) (end 180.8353 119.253) (width 0.254) (layer F.Cu) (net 8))
 (segment (start 179.5145 117.2083) (end 180.8353 118.5291) (width 0.254) (layer F.Cu) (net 8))
 (segment (start 179.5145 116.8019) (end 179.5145 117.3226) (width 0.254) (layer F.Cu) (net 8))
 (segment (start 180.6321 125.2728) (end 180.6956 125.2728) (width 0.254) (layer F.Cu) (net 6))
 (segment (start 182.626 123.3424) (end 182.9308 123.3424) (width 0.254) (layer F.Cu) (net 6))
 (segment (start 180.6956 125.2728) (end 182.626 123.3424) (width 0.254) (layer F.Cu) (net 6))
 (segment (start 182.9308 123.3424) (end 184.0992 123.3424) (width 0.254) (layer F.Cu) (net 6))
 (segment (start 187.5536 123.8885) (end 187.5536 122.6185) (width 0.254) (layer F.Cu) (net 6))
 (segment (start 187.2615 124.1806) (end 187.5536 123.8885) (width 0.254) (layer F.Cu) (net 6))
 (segment (start 184.9374 124.1806) (end 187.2615 124.1806) (width 0.254) (layer F.Cu) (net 6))
 (segment (start 184.0992 123.3424) (end 184.9374 124.1806) (width 0.254) (layer F.Cu) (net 6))
 (segment (start 180.8353 121.158) (end 180.8353 122.7582) (width 0.254) (layer F.Cu) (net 2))
 (segment (start 180.8353 122.7582) (end 180.5432 123.0503) (width 0.254) (layer F.Cu) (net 2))
 (segment (start 177.00244 126.64948) (end 179.42052 126.64948) (width 0.254) (layer F.Cu) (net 2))
 (segment (start 179.61356 123.14428) (end 179.61356 126.45644) (width 0.254) (layer F.Cu) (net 2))
 (segment (start 179.70754 123.0503) (end 179.61356 123.14428) (width 0.254) (layer F.Cu) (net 2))
 (segment (start 179.70754 123.0503) (end 180.5432 123.0503) (width 0.254) (layer F.Cu) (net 2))
 (segment (start 179.61356 126.45644) (end 179.42052 126.64948) (width 0.254) (layer F.Cu) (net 2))
 (segment (start 177.00244 126.64948) (end 176.9745 126.62154) (width 0.254) (layer F.Cu) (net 2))
 (segment (start 176.9745 126.62154) (end 176.9745 125.35662) (width 0.254) (layer F.Cu) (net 2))
 (segment (start 177.00244 126.64948) (end 176.9745 126.62154) (width 0.254) (layer F.Cu) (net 2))
 (segment (start 178.3334 121.2342) (end 180.7591 121.2342) (width 0.254) (layer F.Cu) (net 2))
 (segment (start 180.7591 121.2342) (end 180.8353 121.158) (width 0.254) (layer F.Cu) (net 2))
 (segment (start 180.5432 123.0503) (end 181.1909 123.0503) (width 0.254) (layer F.Cu) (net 2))
 (segment (start 186.38774 122.4153) (end 186.59602 122.62358) (width 0.254) (layer F.Cu) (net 2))
 (segment (start 181.8259 122.4153) (end 186.38774 122.4153) (width 0.254) (layer F.Cu) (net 2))
 (segment (start 181.1909 123.0503) (end 181.8259 122.4153) (width 0.254) (layer F.Cu) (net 2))
 (segment (start 180.467 121.1072) (end 180.5432 121.1834) (width 0.254) (layer F.Cu) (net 2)))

